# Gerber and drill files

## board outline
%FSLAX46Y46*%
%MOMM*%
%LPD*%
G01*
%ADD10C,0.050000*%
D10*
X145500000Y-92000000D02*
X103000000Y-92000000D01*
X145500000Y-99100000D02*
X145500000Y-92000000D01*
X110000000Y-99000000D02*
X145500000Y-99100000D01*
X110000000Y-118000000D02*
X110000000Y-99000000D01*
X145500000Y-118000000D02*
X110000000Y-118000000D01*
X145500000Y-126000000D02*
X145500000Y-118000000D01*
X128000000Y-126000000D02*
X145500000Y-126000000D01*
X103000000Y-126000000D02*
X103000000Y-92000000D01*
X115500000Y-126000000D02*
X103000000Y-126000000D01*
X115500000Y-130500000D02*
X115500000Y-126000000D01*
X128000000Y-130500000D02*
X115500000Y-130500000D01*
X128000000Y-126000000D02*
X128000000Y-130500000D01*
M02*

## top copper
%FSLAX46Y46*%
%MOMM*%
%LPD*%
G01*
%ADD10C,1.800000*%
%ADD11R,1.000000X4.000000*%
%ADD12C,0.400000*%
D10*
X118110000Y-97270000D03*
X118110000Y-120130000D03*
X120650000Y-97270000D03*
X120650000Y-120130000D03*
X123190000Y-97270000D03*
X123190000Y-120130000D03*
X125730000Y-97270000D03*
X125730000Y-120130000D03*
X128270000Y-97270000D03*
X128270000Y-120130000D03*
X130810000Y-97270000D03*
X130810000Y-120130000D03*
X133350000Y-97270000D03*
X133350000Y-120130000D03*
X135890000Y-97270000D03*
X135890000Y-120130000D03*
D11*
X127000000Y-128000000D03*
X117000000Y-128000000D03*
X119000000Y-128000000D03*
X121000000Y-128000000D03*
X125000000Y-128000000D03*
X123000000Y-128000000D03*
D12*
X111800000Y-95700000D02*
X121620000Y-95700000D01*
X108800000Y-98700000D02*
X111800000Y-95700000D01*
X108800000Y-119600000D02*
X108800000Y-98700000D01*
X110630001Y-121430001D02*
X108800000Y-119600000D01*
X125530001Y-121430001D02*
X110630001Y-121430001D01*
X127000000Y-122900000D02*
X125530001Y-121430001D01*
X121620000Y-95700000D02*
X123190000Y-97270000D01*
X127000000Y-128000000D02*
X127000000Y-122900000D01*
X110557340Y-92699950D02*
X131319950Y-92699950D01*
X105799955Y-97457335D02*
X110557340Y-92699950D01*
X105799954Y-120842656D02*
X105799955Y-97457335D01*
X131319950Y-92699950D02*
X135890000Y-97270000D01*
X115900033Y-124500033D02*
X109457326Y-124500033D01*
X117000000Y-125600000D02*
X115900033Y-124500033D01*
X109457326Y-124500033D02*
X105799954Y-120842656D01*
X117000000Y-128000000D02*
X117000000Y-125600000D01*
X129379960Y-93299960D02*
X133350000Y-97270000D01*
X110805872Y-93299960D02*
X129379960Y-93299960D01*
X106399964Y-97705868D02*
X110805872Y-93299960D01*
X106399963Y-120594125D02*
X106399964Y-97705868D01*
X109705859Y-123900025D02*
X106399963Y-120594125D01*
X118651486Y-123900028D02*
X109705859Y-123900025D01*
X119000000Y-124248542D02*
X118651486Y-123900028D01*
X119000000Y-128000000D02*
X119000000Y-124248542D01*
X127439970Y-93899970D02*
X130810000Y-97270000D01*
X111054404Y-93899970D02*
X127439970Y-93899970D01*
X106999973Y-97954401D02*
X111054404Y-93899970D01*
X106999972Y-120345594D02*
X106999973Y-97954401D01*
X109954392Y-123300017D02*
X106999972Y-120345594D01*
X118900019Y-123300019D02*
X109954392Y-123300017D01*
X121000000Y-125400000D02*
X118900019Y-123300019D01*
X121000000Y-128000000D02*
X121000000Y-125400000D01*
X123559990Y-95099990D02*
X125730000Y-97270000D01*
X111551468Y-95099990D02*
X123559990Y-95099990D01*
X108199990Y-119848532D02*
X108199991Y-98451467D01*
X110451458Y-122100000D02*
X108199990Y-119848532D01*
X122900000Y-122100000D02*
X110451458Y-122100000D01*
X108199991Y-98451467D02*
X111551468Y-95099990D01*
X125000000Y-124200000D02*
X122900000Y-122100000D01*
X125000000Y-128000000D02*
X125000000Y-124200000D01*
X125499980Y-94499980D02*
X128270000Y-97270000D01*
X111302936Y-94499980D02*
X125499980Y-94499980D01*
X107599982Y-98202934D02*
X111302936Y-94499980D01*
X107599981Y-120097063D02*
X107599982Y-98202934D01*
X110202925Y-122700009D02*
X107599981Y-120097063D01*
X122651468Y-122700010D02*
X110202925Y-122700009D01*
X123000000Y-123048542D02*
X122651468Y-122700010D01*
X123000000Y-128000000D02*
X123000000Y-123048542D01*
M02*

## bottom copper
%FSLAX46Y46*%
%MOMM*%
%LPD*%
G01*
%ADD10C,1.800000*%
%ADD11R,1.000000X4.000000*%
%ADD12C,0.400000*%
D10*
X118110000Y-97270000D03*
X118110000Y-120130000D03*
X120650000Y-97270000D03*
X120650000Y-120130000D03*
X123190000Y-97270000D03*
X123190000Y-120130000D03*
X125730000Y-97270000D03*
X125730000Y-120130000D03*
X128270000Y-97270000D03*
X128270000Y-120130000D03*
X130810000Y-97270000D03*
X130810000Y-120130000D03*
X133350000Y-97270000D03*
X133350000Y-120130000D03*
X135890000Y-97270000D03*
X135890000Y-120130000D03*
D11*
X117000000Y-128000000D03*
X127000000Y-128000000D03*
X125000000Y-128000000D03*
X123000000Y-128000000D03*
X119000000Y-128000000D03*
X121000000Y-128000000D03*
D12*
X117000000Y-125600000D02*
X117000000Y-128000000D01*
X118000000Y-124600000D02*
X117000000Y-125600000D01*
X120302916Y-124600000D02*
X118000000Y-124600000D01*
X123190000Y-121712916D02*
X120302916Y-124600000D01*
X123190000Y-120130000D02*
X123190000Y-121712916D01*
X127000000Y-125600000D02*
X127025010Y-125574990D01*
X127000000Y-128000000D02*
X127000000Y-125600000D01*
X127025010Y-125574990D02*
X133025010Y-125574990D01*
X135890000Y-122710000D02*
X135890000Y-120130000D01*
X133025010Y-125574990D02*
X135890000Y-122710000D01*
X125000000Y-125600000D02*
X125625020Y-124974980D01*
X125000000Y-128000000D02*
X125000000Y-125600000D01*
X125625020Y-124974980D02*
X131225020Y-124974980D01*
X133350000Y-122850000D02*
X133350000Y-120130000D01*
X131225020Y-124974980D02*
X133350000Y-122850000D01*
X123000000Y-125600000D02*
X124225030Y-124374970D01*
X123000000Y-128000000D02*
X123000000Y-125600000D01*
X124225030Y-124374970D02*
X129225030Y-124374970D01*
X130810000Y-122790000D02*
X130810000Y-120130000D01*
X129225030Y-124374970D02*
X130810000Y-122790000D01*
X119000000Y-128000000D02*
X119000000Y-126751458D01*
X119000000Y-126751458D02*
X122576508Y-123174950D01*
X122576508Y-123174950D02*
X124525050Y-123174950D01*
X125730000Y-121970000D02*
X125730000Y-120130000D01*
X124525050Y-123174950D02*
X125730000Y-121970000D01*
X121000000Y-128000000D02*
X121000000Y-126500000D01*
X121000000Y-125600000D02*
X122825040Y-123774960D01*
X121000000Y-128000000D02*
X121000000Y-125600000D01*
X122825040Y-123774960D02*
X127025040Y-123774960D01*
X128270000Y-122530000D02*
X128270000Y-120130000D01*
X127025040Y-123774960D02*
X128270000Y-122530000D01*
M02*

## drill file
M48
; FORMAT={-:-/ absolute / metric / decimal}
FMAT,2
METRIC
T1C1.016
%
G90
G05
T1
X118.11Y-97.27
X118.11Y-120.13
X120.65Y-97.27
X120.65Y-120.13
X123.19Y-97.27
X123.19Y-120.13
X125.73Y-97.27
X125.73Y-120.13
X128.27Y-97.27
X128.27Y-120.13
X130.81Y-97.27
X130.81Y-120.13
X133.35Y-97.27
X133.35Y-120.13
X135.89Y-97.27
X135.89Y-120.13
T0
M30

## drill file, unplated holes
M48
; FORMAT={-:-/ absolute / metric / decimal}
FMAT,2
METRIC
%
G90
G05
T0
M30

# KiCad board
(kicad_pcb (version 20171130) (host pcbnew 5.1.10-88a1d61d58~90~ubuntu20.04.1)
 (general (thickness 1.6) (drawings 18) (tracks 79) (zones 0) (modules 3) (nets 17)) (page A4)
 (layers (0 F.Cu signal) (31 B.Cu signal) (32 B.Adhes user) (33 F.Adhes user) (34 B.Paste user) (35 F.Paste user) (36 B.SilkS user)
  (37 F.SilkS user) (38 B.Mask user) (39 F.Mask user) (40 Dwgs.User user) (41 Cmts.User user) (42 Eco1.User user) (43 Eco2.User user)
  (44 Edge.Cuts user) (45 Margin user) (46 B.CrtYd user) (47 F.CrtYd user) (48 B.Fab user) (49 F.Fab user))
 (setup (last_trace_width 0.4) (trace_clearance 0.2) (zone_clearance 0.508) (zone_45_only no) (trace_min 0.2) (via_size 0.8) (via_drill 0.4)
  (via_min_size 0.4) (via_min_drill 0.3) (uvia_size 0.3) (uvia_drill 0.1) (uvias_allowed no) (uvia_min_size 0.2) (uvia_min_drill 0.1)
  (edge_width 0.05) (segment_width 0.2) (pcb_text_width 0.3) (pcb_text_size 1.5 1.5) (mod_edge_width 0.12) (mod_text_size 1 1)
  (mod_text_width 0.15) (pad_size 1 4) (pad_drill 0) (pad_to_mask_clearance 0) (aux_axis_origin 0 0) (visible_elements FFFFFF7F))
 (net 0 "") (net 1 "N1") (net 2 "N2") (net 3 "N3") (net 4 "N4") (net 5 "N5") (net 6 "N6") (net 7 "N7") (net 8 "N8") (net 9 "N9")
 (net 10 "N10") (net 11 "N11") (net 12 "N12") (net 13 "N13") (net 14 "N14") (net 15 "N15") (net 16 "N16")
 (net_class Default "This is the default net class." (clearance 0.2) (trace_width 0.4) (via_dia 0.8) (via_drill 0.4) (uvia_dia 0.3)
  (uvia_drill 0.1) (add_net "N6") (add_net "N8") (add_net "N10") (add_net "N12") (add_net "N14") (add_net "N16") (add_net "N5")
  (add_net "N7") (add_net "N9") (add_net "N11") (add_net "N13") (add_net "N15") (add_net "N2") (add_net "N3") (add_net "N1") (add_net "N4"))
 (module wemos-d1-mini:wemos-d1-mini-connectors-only (layer F.Cu) (at 127 108.7 180)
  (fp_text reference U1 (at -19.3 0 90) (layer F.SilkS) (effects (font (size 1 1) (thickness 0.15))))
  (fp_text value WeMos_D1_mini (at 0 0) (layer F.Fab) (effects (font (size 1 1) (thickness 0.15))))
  (pad 16 thru_hole circle (at 8.89 11.43 180) (size 1.8 1.8) (drill 1.016) (layers *.Cu *.Mask) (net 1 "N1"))
  (pad 1 thru_hole circle (at 8.89 -11.43 180) (size 1.8 1.8) (drill 1.016) (layers *.Cu *.Mask) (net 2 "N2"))
  (pad 15 thru_hole circle (at 6.35 11.43 180) (size 1.8 1.8) (drill 1.016) (layers *.Cu *.Mask) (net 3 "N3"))
  (pad 2 thru_hole circle (at 6.35 -11.43 180) (size 1.8 1.8) (drill 1.016) (layers *.Cu *.Mask) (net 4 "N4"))
  (pad 14 thru_hole circle (at 3.81 11.43 180) (size 1.8 1.8) (drill 1.016) (layers *.Cu *.Mask) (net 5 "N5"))
  (pad 3 thru_hole circle (at 3.81 -11.43 180) (size 1.8 1.8) (drill 1.016) (layers *.Cu *.Mask) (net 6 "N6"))
  (pad 13 thru_hole circle (at 1.27 11.43 180) (size 1.8 1.8) (drill 1.016) (layers *.Cu *.Mask) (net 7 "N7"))
  (pad 4 thru_hole circle (at 1.27 -11.43 180) (size 1.8 1.8) (drill 1.016) (layers *.Cu *.Mask) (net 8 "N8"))
  (pad 12 thru_hole circle (at -1.27 11.43 180) (size 1.8 1.8) (drill 1.016) (layers *.Cu *.Mask) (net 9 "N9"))
  (pad 5 thru_hole circle (at -1.27 -11.43 180) (size 1.8 1.8) (drill 1.016) (layers *.Cu *.Mask) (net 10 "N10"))
  (pad 11 thru_hole circle (at -3.81 11.43 180) (size 1.8 1.8) (drill 1.016) (layers *.Cu *.Mask) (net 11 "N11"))
  (pad 6 thru_hole circle (at -3.81 -11.43 180) (size 1.8 1.8) (drill 1.016) (layers *.Cu *.Mask) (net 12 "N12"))
  (pad 10 thru_hole circle (at -6.35 11.43 180) (size 1.8 1.8) (drill 1.016) (layers *.Cu *.Mask) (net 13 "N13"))
  (pad 7 thru_hole circle (at -6.35 -11.43 180) (size 1.8 1.8) (drill 1.016) (layers *.Cu *.Mask) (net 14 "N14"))
  (pad 9 thru_hole circle (at -8.89 11.43 180) (size 1.8 1.8) (drill 1.016) (layers *.Cu *.Mask) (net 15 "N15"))
  (pad 8 thru_hole circle (at -8.89 -11.43 180) (size 1.8 1.8) (drill 1.016) (layers *.Cu *.Mask) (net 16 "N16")))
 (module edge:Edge (layer F.Cu) (at 121 128)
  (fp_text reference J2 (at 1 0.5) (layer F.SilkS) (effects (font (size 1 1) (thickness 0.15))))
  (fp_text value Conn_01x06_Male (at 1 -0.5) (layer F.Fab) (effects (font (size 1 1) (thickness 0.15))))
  (pad 1 connect rect (at 6 0) (size 1 4) (layers F.Cu F.Mask) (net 5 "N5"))
  (pad 6 connect rect (at -4 0) (size 1 4) (layers F.Cu F.Mask) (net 15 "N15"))
  (pad 5 connect rect (at -2 0) (size 1 4) (layers F.Cu F.Mask) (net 13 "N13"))
  (pad 4 connect rect (at 0 0) (size 1 4) (layers F.Cu F.Mask) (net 11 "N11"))
  (pad 2 connect rect (at 4 0) (size 1 4) (layers F.Cu F.Mask) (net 7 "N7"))
  (pad 3 connect rect (at 2 0) (size 1 4) (layers F.Cu F.Mask) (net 9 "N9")))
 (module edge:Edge (layer B.Cu) (at 123 128 180)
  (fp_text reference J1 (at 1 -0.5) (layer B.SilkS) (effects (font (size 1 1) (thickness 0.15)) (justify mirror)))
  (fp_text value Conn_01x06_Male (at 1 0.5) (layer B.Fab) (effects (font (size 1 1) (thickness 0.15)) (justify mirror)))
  (pad 1 connect rect (at 6 0 180) (size 1 4) (layers B.Cu B.Mask) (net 6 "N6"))
  (pad 6 connect rect (at -4 0 180) (size 1 4) (layers B.Cu B.Mask) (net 16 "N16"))
  (pad 5 connect rect (at -2 0 180) (size 1 4) (layers B.Cu B.Mask) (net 14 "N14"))
  (pad 4 connect rect (at 0 0 180) (size 1 4) (layers B.Cu B.Mask) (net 12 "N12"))
  (pad 2 connect rect (at 4 0 180) (size 1 4) (layers B.Cu B.Mask) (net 8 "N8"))
  (pad 3 connect rect (at 2 0 180) (size 1 4) (layers B.Cu B.Mask) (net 10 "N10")))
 (gr_line (start 145.5 92) (end 103 92) (layer Edge.Cuts) (width 0.05))
 (gr_line (start 145.5 99.1) (end 145.5 92) (layer Edge.Cuts) (width 0.05))
 (gr_line (start 110 99) (end 145.5 99.1) (layer Edge.Cuts) (width 0.05))
 (gr_line (start 110 118) (end 110 99) (layer Edge.Cuts) (width 0.05))
 (gr_line (start 145.5 118) (end 110 118) (layer Edge.Cuts) (width 0.05))
 (gr_line (start 145.5 126) (end 145.5 118) (layer Edge.Cuts) (width 0.05))
 (gr_line (start 128 126) (end 145.5 126) (layer Edge.Cuts) (width 0.05))
 (gr_line (start 103 126) (end 103 92) (layer Edge.Cuts) (width 0.05))
 (gr_line (start 115.5 126) (end 103 126) (layer Edge.Cuts) (width 0.05))
 (gr_line (start 115.5 130.5) (end 115.5 126) (layer Edge.Cuts) (width 0.05))
 (gr_line (start 128 130.5) (end 115.5 130.5) (layer Edge.Cuts) (width 0.05))
 (gr_line (start 128 126) (end 128 130.5) (layer Edge.Cuts) (width 0.05))
 (segment (start 117 125.6) (end 117 128) (width 0.4) (layer B.Cu) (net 6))
 (segment (start 118 124.6) (end 117 125.6) (width 0.4) (layer B.Cu) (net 6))
 (segment (start 120.302916 124.6) (end 118 124.6) (width 0.4) (layer B.Cu) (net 6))
 (segment (start 123.19 121.712916) (end 120.302916 124.6) (width 0.4) (layer B.Cu) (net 6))
 (segment (start 123.19 120.13) (end 123.19 121.712916) (width 0.4) (layer B.Cu) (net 6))
 (segment (start 127 125.6) (end 127.02501 125.57499) (width 0.4) (layer B.Cu) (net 16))
 (segment (start 127 128) (end 127 125.6) (width 0.4) (layer B.Cu) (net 16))
 (segment (start 127.02501 125.57499) (end 133.02501 125.57499) (width 0.4) (layer B.Cu) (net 16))
 (segment (start 135.89 122.71) (end 135.89 120.13) (width 0.4) (layer B.Cu) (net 16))
 (segment (start 133.02501 125.57499) (end 135.89 122.71) (width 0.4) (layer B.Cu) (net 16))
 (segment (start 125 125.6) (end 125.62502 124.97498) (width 0.4) (layer B.Cu) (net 14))
 (segment (start 125 128) (end 125 125.6) (width 0.4) (layer B.Cu) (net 14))
 (segment (start 125.62502 124.97498) (end 131.22502 124.97498) (width 0.4) (layer B.Cu) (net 14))
 (segment (start 133.35 122.85) (end 133.35 120.13) (width 0.4) (layer B.Cu) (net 14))
 (segment (start 131.22502 124.97498) (end 133.35 122.85) (width 0.4) (layer B.Cu) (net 14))
 (segment (start 123 125.6) (end 124.22503 124.37497) (width 0.4) (layer B.Cu) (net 12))
 (segment (start 123 128) (end 123 125.6) (width 0.4) (layer B.Cu) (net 12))
 (segment (start 124.22503 124.37497) (end 129.22503 124.37497) (width 0.4) (layer B.Cu) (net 12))
 (segment (start 130.81 122.79) (end 130.81 120.13) (width 0.4) (layer B.Cu) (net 12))
 (segment (start 129.22503 124.37497) (end 130.81 122.79) (width 0.4) (layer B.Cu) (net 12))
 (segment (start 119 128) (end 119 126.751458) (width 0.4) (layer B.Cu) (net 8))
 (segment (start 119 126.751458) (end 122.576508 123.17495) (width 0.4) (layer B.Cu) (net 8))
 (segment (start 122.576508 123.17495) (end 124.52505 123.17495) (width 0.4) (layer B.Cu) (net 8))
 (segment (start 125.73 121.97) (end 125.73 120.13) (width 0.4) (layer B.Cu) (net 8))
 (segment (start 124.52505 123.17495) (end 125.73 121.97) (width 0.4) (layer B.Cu) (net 8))
 (segment (start 121 128) (end 121 126.5) (width 0.4) (layer B.Cu) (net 10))
 (segment (start 121 125.6) (end 122.82504 123.77496) (width 0.4) (layer B.Cu) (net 10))
 (segment (start 121 128) (end 121 125.6) (width 0.4) (layer B.Cu) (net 10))
 (segment (start 122.82504 123.77496) (end 127.02504 123.77496) (width 0.4) (layer B.Cu) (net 10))
 (segment (start 128.27 122.53) (end 128.27 120.13) (width 0.4) (layer B.Cu) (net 10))
 (segment (start 127.02504 123.77496) (end 128.27 122.53) (width 0.4) (layer B.Cu) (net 10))
 (segment (start 111.8 95.7) (end 121.62 95.7) (width 0.4) (layer F.Cu) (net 5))
 (segment (start 108.8 98.7) (end 111.8 95.7) (width 0.4) (layer F.Cu) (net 5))
 (segment (start 108.8 119.6) (end 108.8 98.7) (width 0.4) (layer F.Cu) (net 5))
 (segment (start 110.630001 121.430001) (end 108.8 119.6) (width 0.4) (layer F.Cu) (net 5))
 (segment (start 125.530001 121.430001) (end 110.630001 121.430001) (width 0.4) (layer F.Cu) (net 5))
 (segment (start 127 122.9) (end 125.530001 121.430001) (width 0.4) (layer F.Cu) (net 5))
 (segment (start 121.62 95.7) (end 123.19 97.27) (width 0.4) (layer F.Cu) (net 5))
 (segment (start 127 128) (end 127 122.9) (width 0.4) (layer F.Cu) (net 5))
 (segment (start 110.55734 92.69995) (end 131.31995 92.69995) (width 0.4) (layer F.Cu) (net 15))
 (segment (start 105.799955 97.457335) (end 110.55734 92.69995) (width 0.4) (layer F.Cu) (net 15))
 (segment (start 105.799954 120.842656) (end 105.799955 97.457335) (width 0.4) (layer F.Cu) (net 15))
 (segment (start 131.31995 92.69995) (end 135.89 97.27) (width 0.4) (layer F.Cu) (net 15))
 (segment (start 115.900033 124.500033) (end 109.457326 124.500033) (width 0.4) (layer F.Cu) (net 15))
 (segment (start 117 125.6) (end 115.900033 124.500033) (width 0.4) (layer F.Cu) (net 15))
 (segment (start 109.457326 124.500033) (end 105.799954 120.842656) (width 0.4) (layer F.Cu) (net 15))
 (segment (start 117 128) (end 117 125.6) (width 0.4) (layer F.Cu) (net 15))
 (segment (start 129.37996 93.29996) (end 133.35 97.27) (width 0.4) (layer F.Cu) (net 13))
 (segment (start 110.805872 93.29996) (end 129.37996 93.29996) (width 0.4) (layer F.Cu) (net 13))
 (segment (start 106.399964 97.705868) (end 110.805872 93.29996) (width 0.4) (layer F.Cu) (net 13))
 (segment (start 106.399963 120.594125) (end 106.399964 97.705868) (width 0.4) (layer F.Cu) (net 13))
 (segment (start 109.705859 123.900025) (end 106.399963 120.594125) (width 0.4) (layer F.Cu) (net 13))
 (segment (start 118.651486 123.900028) (end 109.705859 123.900025) (width 0.4) (layer F.Cu) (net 13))
 (segment (start 119 124.248542) (end 118.651486 123.900028) (width 0.4) (layer F.Cu) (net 13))
 (segment (start 119 128) (end 119 124.248542) (width 0.4) (layer F.Cu) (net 13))
 (segment (start 127.43997 93.89997) (end 130.81 97.27) (width 0.4) (layer F.Cu) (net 11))
 (segment (start 111.054404 93.89997) (end 127.43997 93.89997) (width 0.4) (layer F.Cu) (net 11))
 (segment (start 106.999973 97.954401) (end 111.054404 93.89997) (width 0.4) (layer F.Cu) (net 11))
 (segment (start 106.999972 120.345594) (end 106.999973 97.954401) (width 0.4) (layer F.Cu) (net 11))
 (segment (start 109.954392 123.300017) (end 106.999972 120.345594) (width 0.4) (layer F.Cu) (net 11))
 (segment (start 118.900019 123.300019) (end 109.954392 123.300017) (width 0.4) (layer F.Cu) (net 11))
 (segment (start 121 125.4) (end 118.900019 123.300019) (width 0.4) (layer F.Cu) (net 11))
 (segment (start 121 128) (end 121 125.4) (width 0.4) (layer F.Cu) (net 11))
 (segment (start 123.55999 95.09999) (end 125.73 97.27) (width 0.4) (layer F.Cu) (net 7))
 (segment (start 111.551468 95.09999) (end 123.55999 95.09999) (width 0.4) (layer F.Cu) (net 7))
 (segment (start 108.19999 119.848532) (end 108.199991 98.451467) (width 0.4) (layer F.Cu) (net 7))
 (segment (start 110.451458 122.1) (end 108.19999 119.848532) (width 0.4) (layer F.Cu) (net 7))
 (segment (start 122.9 122.1) (end 110.451458 122.1) (width 0.4) (layer F.Cu) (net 7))
 (segment (start 108.199991 98.451467) (end 111.551468 95.09999) (width 0.4) (layer F.Cu) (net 7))
 (segment (start 125 124.2) (end 122.9 122.1) (width 0.4) (layer F.Cu) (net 7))
 (segment (start 125 128) (end 125 124.2) (width 0.4) (layer F.Cu) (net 7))
 (segment (start 125.49998 94.49998) (end 128.27 97.27) (width 0.4) (layer F.Cu) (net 9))
 (segment (start 111.302936 94.49998) (end 125.49998 94.49998) (width 0.4) (layer F.Cu) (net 9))
 (segment (start 107.599982 98.202934) (end 111.302936 94.49998) (width 0.4) (layer F.Cu) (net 9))
 (segment (start 107.599981 120.097063) (end 107.599982 98.202934) (width 0.4) (layer F.Cu) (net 9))
 (segment (start 110.202925 122.700009) (end 107.599981 120.097063) (width 0.4) (layer F.Cu) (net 9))
 (segment (start 122.651468 122.70001) (end 110.202925 122.700009) (width 0.4) (layer F.Cu) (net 9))
 (segment (start 123 123.048542) (end 122.651468 122.70001) (width 0.4) (layer F.Cu) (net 9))
 (segment (start 123 128) (end 123 123.048542) (width 0.4) (layer F.Cu) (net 9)))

